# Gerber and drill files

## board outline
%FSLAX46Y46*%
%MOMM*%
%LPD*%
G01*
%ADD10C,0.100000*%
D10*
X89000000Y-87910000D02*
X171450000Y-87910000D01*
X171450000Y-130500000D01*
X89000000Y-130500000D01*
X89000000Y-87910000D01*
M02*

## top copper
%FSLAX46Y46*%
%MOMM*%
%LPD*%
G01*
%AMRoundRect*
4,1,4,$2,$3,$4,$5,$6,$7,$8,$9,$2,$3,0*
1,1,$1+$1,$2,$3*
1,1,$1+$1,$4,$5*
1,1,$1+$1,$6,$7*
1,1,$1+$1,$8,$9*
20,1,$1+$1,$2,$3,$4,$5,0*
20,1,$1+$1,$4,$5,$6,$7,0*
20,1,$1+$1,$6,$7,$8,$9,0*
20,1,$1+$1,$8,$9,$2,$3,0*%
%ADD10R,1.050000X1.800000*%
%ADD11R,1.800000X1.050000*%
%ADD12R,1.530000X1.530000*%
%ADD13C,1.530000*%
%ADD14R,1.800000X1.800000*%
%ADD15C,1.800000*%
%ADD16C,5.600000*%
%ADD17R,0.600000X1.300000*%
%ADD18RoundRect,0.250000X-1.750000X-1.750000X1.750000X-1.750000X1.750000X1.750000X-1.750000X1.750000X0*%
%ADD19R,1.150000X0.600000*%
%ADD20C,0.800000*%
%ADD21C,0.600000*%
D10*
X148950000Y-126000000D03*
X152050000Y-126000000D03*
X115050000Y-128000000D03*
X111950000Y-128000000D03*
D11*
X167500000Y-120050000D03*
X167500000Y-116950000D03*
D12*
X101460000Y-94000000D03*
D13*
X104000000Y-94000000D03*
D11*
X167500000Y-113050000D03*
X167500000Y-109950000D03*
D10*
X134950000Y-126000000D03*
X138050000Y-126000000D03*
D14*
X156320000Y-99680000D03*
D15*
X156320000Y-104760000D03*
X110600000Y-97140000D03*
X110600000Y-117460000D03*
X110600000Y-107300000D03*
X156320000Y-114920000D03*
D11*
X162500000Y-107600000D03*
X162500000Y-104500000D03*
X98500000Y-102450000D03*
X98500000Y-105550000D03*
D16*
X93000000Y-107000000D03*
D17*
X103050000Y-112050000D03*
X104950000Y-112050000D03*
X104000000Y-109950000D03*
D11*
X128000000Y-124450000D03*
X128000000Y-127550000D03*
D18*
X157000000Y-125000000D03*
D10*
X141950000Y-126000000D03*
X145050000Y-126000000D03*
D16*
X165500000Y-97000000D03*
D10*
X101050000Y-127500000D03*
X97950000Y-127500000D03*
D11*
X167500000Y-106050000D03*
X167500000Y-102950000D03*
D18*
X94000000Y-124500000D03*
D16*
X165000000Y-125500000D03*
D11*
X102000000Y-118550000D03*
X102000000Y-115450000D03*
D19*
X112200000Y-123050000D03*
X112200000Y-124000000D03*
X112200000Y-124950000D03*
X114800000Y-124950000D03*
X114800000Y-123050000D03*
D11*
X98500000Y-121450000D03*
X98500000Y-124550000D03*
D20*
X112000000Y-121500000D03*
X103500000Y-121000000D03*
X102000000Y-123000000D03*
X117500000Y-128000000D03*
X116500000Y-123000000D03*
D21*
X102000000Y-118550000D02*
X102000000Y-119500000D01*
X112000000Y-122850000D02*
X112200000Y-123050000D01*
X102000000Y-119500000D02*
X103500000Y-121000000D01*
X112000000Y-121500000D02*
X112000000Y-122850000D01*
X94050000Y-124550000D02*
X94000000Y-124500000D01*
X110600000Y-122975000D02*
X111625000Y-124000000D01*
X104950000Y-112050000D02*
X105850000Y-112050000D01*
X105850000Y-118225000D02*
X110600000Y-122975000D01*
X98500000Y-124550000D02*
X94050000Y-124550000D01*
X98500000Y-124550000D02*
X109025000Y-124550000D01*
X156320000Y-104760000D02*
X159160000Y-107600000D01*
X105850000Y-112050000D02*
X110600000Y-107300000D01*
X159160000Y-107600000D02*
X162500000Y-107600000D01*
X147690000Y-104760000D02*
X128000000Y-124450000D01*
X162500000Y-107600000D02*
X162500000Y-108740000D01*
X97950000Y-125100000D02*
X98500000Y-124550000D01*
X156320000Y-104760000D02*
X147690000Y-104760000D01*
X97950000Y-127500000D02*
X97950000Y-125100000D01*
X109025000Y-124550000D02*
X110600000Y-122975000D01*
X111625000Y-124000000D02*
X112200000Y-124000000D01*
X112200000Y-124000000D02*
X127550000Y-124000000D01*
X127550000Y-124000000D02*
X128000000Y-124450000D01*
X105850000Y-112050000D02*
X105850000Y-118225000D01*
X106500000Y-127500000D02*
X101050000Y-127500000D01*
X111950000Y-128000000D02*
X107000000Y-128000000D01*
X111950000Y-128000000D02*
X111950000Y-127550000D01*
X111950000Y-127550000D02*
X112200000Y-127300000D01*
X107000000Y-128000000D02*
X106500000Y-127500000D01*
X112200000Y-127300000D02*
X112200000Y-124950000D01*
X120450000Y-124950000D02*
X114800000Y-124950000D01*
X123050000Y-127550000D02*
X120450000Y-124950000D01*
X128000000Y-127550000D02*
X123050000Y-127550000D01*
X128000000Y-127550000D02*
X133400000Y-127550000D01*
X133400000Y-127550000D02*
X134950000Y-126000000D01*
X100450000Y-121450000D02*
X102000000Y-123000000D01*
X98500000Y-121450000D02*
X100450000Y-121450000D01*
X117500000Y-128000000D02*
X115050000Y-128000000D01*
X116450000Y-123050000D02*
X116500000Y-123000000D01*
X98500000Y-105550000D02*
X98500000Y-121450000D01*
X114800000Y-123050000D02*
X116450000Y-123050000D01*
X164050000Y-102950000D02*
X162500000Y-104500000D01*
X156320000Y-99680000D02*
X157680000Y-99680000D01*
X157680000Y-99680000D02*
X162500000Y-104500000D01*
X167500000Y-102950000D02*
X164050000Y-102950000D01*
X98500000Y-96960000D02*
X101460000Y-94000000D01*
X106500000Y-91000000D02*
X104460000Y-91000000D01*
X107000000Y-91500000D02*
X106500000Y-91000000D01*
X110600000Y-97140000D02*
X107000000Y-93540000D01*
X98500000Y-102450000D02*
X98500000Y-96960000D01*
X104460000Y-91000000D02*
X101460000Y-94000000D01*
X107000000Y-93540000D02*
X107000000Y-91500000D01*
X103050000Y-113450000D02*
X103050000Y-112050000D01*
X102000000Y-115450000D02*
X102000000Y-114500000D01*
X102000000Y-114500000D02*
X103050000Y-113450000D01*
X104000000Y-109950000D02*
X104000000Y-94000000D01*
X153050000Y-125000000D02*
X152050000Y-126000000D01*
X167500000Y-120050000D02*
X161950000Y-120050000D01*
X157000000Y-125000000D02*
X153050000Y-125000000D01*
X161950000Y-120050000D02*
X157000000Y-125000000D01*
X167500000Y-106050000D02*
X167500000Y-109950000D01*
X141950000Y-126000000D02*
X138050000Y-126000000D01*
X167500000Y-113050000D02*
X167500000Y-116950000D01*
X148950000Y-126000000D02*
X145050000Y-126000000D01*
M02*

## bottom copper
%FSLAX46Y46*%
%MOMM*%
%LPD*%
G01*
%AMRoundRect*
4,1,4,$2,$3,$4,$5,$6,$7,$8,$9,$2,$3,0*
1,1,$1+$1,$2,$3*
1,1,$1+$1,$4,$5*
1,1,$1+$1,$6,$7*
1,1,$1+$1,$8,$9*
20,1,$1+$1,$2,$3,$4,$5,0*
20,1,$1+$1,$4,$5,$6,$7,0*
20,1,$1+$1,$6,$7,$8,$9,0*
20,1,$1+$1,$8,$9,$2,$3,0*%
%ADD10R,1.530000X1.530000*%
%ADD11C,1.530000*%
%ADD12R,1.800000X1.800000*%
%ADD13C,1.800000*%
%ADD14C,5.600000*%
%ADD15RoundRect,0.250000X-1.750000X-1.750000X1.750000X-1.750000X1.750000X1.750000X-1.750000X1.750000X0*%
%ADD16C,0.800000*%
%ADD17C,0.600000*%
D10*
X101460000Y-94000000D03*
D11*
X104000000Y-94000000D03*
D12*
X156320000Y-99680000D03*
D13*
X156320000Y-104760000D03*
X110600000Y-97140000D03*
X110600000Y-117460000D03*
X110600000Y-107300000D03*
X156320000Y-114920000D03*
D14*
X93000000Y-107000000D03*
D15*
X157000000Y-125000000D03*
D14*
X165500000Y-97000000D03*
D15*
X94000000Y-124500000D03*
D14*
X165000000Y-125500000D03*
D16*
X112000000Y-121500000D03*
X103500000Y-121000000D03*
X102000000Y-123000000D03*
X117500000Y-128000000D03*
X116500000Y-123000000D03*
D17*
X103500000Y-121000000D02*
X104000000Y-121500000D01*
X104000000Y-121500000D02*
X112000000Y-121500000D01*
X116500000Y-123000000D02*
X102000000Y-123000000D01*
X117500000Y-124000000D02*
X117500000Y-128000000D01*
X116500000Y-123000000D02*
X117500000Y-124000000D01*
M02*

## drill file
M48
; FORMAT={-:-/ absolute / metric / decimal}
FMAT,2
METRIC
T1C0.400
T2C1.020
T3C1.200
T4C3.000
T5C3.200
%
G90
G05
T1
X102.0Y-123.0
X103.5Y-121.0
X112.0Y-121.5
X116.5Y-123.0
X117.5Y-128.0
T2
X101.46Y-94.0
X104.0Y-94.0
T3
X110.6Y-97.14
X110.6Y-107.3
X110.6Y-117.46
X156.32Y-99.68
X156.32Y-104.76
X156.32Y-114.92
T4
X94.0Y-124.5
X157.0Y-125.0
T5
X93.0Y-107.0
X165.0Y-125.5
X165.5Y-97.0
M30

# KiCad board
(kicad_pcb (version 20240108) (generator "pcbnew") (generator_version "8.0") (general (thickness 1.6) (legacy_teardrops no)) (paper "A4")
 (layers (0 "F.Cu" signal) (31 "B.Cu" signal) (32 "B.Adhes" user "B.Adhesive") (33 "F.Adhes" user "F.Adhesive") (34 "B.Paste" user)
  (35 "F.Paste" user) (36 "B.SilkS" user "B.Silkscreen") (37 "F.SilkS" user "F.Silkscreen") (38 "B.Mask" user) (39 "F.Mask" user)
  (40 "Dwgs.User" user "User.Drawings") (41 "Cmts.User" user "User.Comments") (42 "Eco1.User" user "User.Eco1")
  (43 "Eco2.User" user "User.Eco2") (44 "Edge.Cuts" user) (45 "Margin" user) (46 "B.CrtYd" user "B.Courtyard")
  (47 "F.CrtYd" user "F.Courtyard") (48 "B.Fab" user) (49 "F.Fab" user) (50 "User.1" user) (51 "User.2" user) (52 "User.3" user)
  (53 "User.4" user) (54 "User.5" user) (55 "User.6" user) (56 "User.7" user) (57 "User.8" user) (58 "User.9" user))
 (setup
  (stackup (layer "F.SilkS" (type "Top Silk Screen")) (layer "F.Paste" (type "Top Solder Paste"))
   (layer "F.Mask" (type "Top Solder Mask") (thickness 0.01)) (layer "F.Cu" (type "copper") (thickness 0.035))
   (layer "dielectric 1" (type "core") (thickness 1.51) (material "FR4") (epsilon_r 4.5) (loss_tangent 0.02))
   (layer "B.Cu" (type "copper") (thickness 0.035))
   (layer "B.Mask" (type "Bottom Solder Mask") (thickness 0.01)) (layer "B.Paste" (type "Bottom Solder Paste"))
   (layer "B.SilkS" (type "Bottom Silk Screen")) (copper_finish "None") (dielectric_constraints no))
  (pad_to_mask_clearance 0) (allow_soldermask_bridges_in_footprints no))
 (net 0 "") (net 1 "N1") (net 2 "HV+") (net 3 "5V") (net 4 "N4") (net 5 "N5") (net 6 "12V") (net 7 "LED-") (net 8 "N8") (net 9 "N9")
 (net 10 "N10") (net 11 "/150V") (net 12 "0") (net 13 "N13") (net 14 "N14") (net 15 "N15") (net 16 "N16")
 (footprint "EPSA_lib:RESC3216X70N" (layer "F.Cu") (at 150.5 126)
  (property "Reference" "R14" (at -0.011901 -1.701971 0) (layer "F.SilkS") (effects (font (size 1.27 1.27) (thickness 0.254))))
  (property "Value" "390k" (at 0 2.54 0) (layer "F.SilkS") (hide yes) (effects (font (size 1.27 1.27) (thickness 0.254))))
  (pad "1" smd rect (at -1.55 0) (size 1.05 1.8) (layers "F.Cu" "F.Paste" "F.Mask") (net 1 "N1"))
  (pad "2" smd rect (at 1.55 0) (size 1.05 1.8) (layers "F.Cu" "F.Paste" "F.Mask") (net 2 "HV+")))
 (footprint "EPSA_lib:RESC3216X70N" (layer "F.Cu") (at 113.5 128 180)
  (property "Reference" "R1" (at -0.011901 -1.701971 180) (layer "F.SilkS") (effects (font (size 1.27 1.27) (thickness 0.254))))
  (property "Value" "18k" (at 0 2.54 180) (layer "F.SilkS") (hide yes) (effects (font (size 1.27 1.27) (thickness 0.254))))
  (pad "1" smd rect (at -1.55 0 180) (size 1.05 1.8) (layers "F.Cu" "F.Paste" "F.Mask") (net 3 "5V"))
  (pad "2" smd rect (at 1.55 0 180) (size 1.05 1.8) (layers "F.Cu" "F.Paste" "F.Mask") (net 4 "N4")))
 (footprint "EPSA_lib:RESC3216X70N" (layer "F.Cu") (at 167.5 118.5 90)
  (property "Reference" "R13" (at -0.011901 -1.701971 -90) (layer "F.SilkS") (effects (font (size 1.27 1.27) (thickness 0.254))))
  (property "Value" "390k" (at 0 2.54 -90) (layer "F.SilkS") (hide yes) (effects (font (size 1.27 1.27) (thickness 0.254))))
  (pad "1" smd rect (at -1.55 0 90) (size 1.05 1.8) (layers "F.Cu" "F.Paste" "F.Mask") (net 2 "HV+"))
  (pad "2" smd rect (at 1.55 0 90) (size 1.05 1.8) (layers "F.Cu" "F.Paste" "F.Mask") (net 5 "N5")))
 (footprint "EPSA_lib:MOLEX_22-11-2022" (layer "F.Cu") (at 101.46 94)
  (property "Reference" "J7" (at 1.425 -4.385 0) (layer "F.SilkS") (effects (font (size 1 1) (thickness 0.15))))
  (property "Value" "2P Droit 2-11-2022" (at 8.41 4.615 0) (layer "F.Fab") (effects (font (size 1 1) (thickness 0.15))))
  (pad "1" thru_hole rect (at 0 0) (size 1.53 1.53) (drill 1.02) (layers "*.Cu" "*.Mask") (remove_unused_layers no) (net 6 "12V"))
  (pad "2" thru_hole circle (at 2.54 0) (size 1.53 1.53) (drill 1.02) (layers "*.Cu" "*.Mask") (remove_unused_layers no) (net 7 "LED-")))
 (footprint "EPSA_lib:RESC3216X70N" (layer "F.Cu") (at 167.5 111.5 90)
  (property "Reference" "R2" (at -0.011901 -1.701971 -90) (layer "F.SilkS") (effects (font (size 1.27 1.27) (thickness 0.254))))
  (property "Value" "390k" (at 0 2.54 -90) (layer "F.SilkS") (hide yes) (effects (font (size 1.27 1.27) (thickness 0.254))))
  (pad "1" smd rect (at -1.55 0 90) (size 1.05 1.8) (layers "F.Cu" "F.Paste" "F.Mask") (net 5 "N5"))
  (pad "2" smd rect (at 1.55 0 90) (size 1.05 1.8) (layers "F.Cu" "F.Paste" "F.Mask") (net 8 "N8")))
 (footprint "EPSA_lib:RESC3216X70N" (layer "F.Cu") (at 136.5 126)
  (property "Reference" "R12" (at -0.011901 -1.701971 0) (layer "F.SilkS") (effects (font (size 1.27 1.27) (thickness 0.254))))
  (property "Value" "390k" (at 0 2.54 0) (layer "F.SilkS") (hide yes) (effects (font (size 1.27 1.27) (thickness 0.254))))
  (pad "1" smd rect (at -1.55 0) (size 1.05 1.8) (layers "F.Cu" "F.Paste" "F.Mask") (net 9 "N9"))
  (pad "2" smd rect (at 1.55 0) (size 1.05 1.8) (layers "F.Cu" "F.Paste" "F.Mask") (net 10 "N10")))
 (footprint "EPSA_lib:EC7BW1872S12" (layer "F.Cu") (at 140.82 130.18 180)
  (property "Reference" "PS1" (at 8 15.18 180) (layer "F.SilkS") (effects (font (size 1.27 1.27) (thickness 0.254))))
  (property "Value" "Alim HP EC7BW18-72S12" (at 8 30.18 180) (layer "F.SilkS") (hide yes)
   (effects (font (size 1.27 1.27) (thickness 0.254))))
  (pad "1" thru_hole rect (at -15.5 30.5 270) (size 1.8 1.8) (drill 1.2) (layers "*.Cu" "*.Mask") (remove_unused_layers no) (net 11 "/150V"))
  (pad "2" thru_hole circle (at -15.5 25.42 270) (size 1.8 1.8) (drill 1.2) (layers "*.Cu" "*.Mask") (remove_unused_layers no) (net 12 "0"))
  (pad "3" thru_hole circle (at 30.22 33.04 270) (size 1.8 1.8) (drill 1.2) (layers "*.Cu" "*.Mask") (remove_unused_layers no) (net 6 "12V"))
  (pad "4" thru_hole circle (at 30.22 12.72 270) (size 1.8 1.8) (drill 1.2) (layers "*.Cu" "*.Mask") (remove_unused_layers no)
   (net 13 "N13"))
  (pad "5" thru_hole circle (at 30.22 22.88 270) (size 1.8 1.8) (drill 1.2) (layers "*.Cu" "*.Mask") (remove_unused_layers no) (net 12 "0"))
  (pad "6" thru_hole circle (at -15.5 15.26 270) (size 1.8 1.8) (drill 1.2) (layers "*.Cu" "*.Mask") (remove_unused_layers no)
   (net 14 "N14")))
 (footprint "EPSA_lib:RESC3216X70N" (layer "F.Cu") (at 162.5 106.05 90)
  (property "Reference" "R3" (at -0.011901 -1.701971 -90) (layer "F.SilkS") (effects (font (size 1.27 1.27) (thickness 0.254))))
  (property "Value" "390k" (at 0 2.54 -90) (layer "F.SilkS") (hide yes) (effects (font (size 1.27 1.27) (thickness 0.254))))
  (pad "1" smd rect (at -1.55 0 90) (size 1.05 1.8) (layers "F.Cu" "F.Paste" "F.Mask") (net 12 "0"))
  (pad "2" smd rect (at 1.55 0 90) (size 1.05 1.8) (layers "F.Cu" "F.Paste" "F.Mask") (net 11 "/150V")))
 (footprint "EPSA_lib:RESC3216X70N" (layer "F.Cu") (at 98.5 104 -90)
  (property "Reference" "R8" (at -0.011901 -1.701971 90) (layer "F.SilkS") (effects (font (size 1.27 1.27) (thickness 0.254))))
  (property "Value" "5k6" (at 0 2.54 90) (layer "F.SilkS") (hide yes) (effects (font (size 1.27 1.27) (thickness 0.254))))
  (pad "1" smd rect (at -1.55 0 270) (size 1.05 1.8) (layers "F.Cu" "F.Paste" "F.Mask") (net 6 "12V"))
  (pad "2" smd rect (at 1.55 0 270) (size 1.05 1.8) (layers "F.Cu" "F.Paste" "F.Mask") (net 3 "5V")))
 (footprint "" (layer "F.Cu") (at 93 107)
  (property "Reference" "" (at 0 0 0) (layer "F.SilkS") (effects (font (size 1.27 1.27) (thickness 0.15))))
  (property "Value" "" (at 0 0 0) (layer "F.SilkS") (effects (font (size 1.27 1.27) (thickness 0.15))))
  (pad "1" thru_hole circle (at 0 0) (size 5.6 5.6) (drill 3.2) (layers "*.Cu" "*.Mask") (remove_unused_layers no)))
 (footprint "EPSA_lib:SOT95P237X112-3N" (layer "F.Cu") (at 104 111 90)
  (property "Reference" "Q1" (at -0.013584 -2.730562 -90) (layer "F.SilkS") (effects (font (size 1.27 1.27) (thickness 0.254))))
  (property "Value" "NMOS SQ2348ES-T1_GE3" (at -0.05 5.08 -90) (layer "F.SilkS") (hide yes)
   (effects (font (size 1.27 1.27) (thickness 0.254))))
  (pad "1" smd rect (at -1.05 -0.95 180) (size 0.6 1.3) (layers "F.Cu" "F.Paste" "F.Mask") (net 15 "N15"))
  (pad "2" smd rect (at -1.05 0.95 180) (size 0.6 1.3) (layers "F.Cu" "F.Paste" "F.Mask") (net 12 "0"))
  (pad "3" smd rect (at 1.05 0 180) (size 0.6 1.3) (layers "F.Cu" "F.Paste" "F.Mask") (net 7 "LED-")))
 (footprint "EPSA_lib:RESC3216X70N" (layer "F.Cu") (at 128 126 -90)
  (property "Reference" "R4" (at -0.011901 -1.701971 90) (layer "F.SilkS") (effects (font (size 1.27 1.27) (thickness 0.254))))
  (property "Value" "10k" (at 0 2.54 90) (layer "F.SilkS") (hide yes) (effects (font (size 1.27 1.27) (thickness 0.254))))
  (pad "1" smd rect (at -1.55 0 270) (size 1.05 1.8) (layers "F.Cu" "F.Paste" "F.Mask") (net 12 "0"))
  (pad "2" smd rect (at 1.55 0 270) (size 1.05 1.8) (layers "F.Cu" "F.Paste" "F.Mask") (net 9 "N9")))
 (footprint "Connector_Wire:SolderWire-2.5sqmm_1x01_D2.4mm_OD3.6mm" (layer "F.Cu") (at 157 125)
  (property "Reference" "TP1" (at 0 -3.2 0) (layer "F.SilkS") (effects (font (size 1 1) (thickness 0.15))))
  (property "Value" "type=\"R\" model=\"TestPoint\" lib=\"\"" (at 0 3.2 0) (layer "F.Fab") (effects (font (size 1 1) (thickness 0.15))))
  (pad "1" thru_hole roundrect (at 0 0) (size 4 4) (drill 3) (layers "*.Cu" "*.Mask") (remove_unused_layers no) (roundrect_rratio 0.0625)
   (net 2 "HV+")))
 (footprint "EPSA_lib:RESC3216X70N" (layer "F.Cu") (at 143.5 126)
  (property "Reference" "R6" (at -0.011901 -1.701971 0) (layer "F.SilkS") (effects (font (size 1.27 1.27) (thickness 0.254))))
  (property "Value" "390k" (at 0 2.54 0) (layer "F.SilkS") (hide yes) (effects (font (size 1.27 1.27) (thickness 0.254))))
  (pad "1" smd rect (at -1.55 0) (size 1.05 1.8) (layers "F.Cu" "F.Paste" "F.Mask") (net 10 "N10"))
  (pad "2" smd rect (at 1.55 0) (size 1.05 1.8) (layers "F.Cu" "F.Paste" "F.Mask") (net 1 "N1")))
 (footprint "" (layer "F.Cu") (at 165.5 97)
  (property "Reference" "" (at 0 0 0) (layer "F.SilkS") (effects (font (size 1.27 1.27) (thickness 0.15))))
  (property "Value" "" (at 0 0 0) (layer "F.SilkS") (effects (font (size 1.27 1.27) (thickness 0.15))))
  (pad "1" thru_hole circle (at 0 0) (size 5.6 5.6) (drill 3.2) (layers "*.Cu" "*.Mask") (remove_unused_layers no)))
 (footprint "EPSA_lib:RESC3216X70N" (layer "F.Cu") (at 99.5 127.5 180)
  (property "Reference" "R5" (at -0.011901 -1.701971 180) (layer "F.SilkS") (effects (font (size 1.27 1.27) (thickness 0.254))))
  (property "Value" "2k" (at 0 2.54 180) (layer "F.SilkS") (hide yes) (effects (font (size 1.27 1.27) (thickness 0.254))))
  (pad "1" smd rect (at -1.55 0 180) (size 1.05 1.8) (layers "F.Cu" "F.Paste" "F.Mask") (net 4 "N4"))
  (pad "2" smd rect (at 1.55 0 180) (size 1.05 1.8) (layers "F.Cu" "F.Paste" "F.Mask") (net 12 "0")))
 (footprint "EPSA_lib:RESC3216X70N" (layer "F.Cu") (at 167.5 104.5 90)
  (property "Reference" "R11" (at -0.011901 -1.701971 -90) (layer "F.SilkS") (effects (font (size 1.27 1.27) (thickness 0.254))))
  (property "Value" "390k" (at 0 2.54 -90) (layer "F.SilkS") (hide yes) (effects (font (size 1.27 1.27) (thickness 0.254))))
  (pad "1" smd rect (at -1.55 0 90) (size 1.05 1.8) (layers "F.Cu" "F.Paste" "F.Mask") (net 8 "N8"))
  (pad "2" smd rect (at 1.55 0 90) (size 1.05 1.8) (layers "F.Cu" "F.Paste" "F.Mask") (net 11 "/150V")))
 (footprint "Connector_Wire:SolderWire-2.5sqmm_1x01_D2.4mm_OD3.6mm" (layer "F.Cu") (at 94 124.5)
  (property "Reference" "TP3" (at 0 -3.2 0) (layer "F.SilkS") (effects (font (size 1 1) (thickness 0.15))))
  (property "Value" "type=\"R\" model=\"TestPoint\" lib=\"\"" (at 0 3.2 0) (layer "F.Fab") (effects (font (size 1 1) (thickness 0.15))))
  (pad "1" thru_hole roundrect (at 0 0) (size 4 4) (drill 3) (layers "*.Cu" "*.Mask") (remove_unused_layers no) (roundrect_rratio 0.0625)
   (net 12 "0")))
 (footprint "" (layer "F.Cu") (at 165 125.5)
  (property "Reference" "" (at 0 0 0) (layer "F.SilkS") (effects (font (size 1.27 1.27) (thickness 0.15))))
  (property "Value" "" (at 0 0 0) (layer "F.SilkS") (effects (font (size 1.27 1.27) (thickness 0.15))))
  (pad "1" thru_hole circle (at 0 0) (size 5.6 5.6) (drill 3.2) (layers "*.Cu" "*.Mask") (remove_unused_layers no)))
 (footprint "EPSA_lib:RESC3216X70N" (layer "F.Cu") (at 102 117 90)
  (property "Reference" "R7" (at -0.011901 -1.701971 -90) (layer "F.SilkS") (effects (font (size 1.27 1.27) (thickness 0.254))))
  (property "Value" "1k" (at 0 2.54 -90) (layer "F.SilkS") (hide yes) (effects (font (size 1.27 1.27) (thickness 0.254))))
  (pad "1" smd rect (at -1.55 0 90) (size 1.05 1.8) (layers "F.Cu" "F.Paste" "F.Mask") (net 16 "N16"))
  (pad "2" smd rect (at 1.55 0 90) (size 1.05 1.8) (layers "F.Cu" "F.Paste" "F.Mask") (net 15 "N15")))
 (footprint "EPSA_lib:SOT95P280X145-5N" (layer "F.Cu") (at 113.5 124)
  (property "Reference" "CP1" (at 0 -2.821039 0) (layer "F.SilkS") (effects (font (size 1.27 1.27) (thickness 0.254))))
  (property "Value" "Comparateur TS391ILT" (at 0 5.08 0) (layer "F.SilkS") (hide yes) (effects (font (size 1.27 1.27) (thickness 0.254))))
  (pad "1" smd rect (at -1.3 -0.95 90) (size 0.6 1.15) (layers "F.Cu" "F.Paste" "F.Mask") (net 16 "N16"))
  (pad "2" smd rect (at -1.3 0 90) (size 0.6 1.15) (layers "F.Cu" "F.Paste" "F.Mask") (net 12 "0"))
  (pad "3" smd rect (at -1.3 0.95 90) (size 0.6 1.15) (layers "F.Cu" "F.Paste" "F.Mask") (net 4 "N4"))
  (pad "4" smd rect (at 1.3 0.95 90) (size 0.6 1.15) (layers "F.Cu" "F.Paste" "F.Mask") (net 9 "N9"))
  (pad "5" smd rect (at 1.3 -0.95 90) (size 0.6 1.15) (layers "F.Cu" "F.Paste" "F.Mask") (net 3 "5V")))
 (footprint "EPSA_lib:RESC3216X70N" (layer "F.Cu") (at 98.5 123 -90)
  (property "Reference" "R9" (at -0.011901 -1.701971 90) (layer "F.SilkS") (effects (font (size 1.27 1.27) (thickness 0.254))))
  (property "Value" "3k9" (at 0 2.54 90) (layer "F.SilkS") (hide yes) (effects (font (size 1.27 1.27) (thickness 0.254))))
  (pad "1" smd rect (at -1.55 0 270) (size 1.05 1.8) (layers "F.Cu" "F.Paste" "F.Mask") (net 3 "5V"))
  (pad "2" smd rect (at 1.55 0 270) (size 1.05 1.8) (layers "F.Cu" "F.Paste" "F.Mask") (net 12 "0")))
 (gr_rect (start 89 87.91) (end 171.45 130.5) (stroke (width 0.1) (type default)) (fill none) (layer "Edge.Cuts"))
 (segment (start 102 118.55) (end 102 119.5) (width 0.6) (layer "F.Cu") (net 16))
 (segment (start 112 122.85) (end 112.2 123.05) (width 0.6) (layer "F.Cu") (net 16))
 (segment (start 102 119.5) (end 103.5 121) (width 0.6) (layer "F.Cu") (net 16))
 (segment (start 112 121.5) (end 112 122.85) (width 0.6) (layer "F.Cu") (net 16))
 (via (at 112 121.5) (size 0.8) (drill 0.4) (layers "F.Cu" "B.Cu") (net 16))
 (via (at 103.5 121) (size 0.8) (drill 0.4) (layers "F.Cu" "B.Cu") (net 16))
 (segment (start 103.5 121) (end 104 121.5) (width 0.6) (layer "B.Cu") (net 16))
 (segment (start 104 121.5) (end 112 121.5) (width 0.6) (layer "B.Cu") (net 16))
 (segment (start 94.05 124.55) (end 94 124.5) (width 0.6) (layer "F.Cu") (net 12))
 (segment (start 110.6 122.975) (end 111.625 124) (width 0.6) (layer "F.Cu") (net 12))
 (segment (start 104.95 112.05) (end 105.85 112.05) (width 0.6) (layer "F.Cu") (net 12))
 (segment (start 105.85 118.225) (end 110.6 122.975) (width 0.6) (layer "F.Cu") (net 12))
 (segment (start 98.5 124.55) (end 94.05 124.55) (width 0.6) (layer "F.Cu") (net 12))
 (segment (start 98.5 124.55) (end 109.025 124.55) (width 0.6) (layer "F.Cu") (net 12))
 (segment (start 156.32 104.76) (end 159.16 107.6) (width 0.6) (layer "F.Cu") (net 12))
 (segment (start 105.85 112.05) (end 110.6 107.3) (width 0.6) (layer "F.Cu") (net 12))
 (segment (start 159.16 107.6) (end 162.5 107.6) (width 0.6) (layer "F.Cu") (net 12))
 (segment (start 147.69 104.76) (end 128 124.45) (width 0.6) (layer "F.Cu") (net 12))
 (segment (start 162.5 107.6) (end 162.5 108.74) (width 0.6) (layer "F.Cu") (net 12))
 (segment (start 97.95 125.1) (end 98.5 124.55) (width 0.6) (layer "F.Cu") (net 12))
 (segment (start 156.32 104.76) (end 147.69 104.76) (width 0.6) (layer "F.Cu") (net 12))
 (segment (start 97.95 127.5) (end 97.95 125.1) (width 0.6) (layer "F.Cu") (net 12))
 (segment (start 109.025 124.55) (end 110.6 122.975) (width 0.6) (layer "F.Cu") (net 12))
 (segment (start 111.625 124) (end 112.2 124) (width 0.6) (layer "F.Cu") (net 12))
 (segment (start 112.2 124) (end 127.55 124) (width 0.6) (layer "F.Cu") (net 12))
 (segment (start 127.55 124) (end 128 124.45) (width 0.6) (layer "F.Cu") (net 12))
 (segment (start 105.85 112.05) (end 105.85 118.225) (width 0.6) (layer "F.Cu") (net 12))
 (segment (start 106.5 127.5) (end 101.05 127.5) (width 0.6) (layer "F.Cu") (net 4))
 (segment (start 111.95 128) (end 107 128) (width 0.6) (layer "F.Cu") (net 4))
 (segment (start 111.95 128) (end 111.95 127.55) (width 0.6) (layer "F.Cu") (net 4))
 (segment (start 111.95 127.55) (end 112.2 127.3) (width 0.6) (layer "F.Cu") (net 4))
 (segment (start 107 128) (end 106.5 127.5) (width 0.6) (layer "F.Cu") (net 4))
 (segment (start 112.2 127.3) (end 112.2 124.95) (width 0.6) (layer "F.Cu") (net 4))
 (segment (start 120.45 124.95) (end 114.8 124.95) (width 0.6) (layer "F.Cu") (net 9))
 (segment (start 123.05 127.55) (end 120.45 124.95) (width 0.6) (layer "F.Cu") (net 9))
 (segment (start 128 127.55) (end 123.05 127.55) (width 0.6) (layer "F.Cu") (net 9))
 (segment (start 128 127.55) (end 133.4 127.55) (width 0.6) (layer "F.Cu") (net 9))
 (segment (start 133.4 127.55) (end 134.95 126) (width 0.6) (layer "F.Cu") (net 9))
 (segment (start 100.45 121.45) (end 102 123) (width 0.6) (layer "F.Cu") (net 3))
 (segment (start 98.5 121.45) (end 100.45 121.45) (width 0.6) (layer "F.Cu") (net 3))
 (segment (start 117.5 128) (end 115.05 128) (width 0.6) (layer "F.Cu") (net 3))
 (segment (start 116.45 123.05) (end 116.5 123) (width 0.6) (layer "F.Cu") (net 3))
 (segment (start 98.5 105.55) (end 98.5 121.45) (width 0.6) (layer "F.Cu") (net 3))
 (segment (start 114.8 123.05) (end 116.45 123.05) (width 0.6) (layer "F.Cu") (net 3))
 (via (at 102 123) (size 0.8) (drill 0.4) (layers "F.Cu" "B.Cu") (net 3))
 (via (at 117.5 128) (size 0.8) (drill 0.4) (layers "F.Cu" "B.Cu") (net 3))
 (via (at 116.5 123) (size 0.8) (drill 0.4) (layers "F.Cu" "B.Cu") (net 3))
 (segment (start 116.5 123) (end 102 123) (width 0.6) (layer "B.Cu") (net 3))
 (segment (start 117.5 124) (end 117.5 128) (width 0.6) (layer "B.Cu") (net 3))
 (segment (start 116.5 123) (end 117.5 124) (width 0.6) (layer "B.Cu") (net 3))
 (segment (start 164.05 102.95) (end 162.5 104.5) (width 0.6) (layer "F.Cu") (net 11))
 (segment (start 156.32 99.68) (end 157.68 99.68) (width 0.6) (layer "F.Cu") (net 11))
 (segment (start 157.68 99.68) (end 162.5 104.5) (width 0.6) (layer "F.Cu") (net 11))
 (segment (start 167.5 102.95) (end 164.05 102.95) (width 0.6) (layer "F.Cu") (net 11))
 (segment (start 98.5 96.96) (end 101.46 94) (width 0.6) (layer "F.Cu") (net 6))
 (segment (start 106.5 91) (end 104.46 91) (width 0.6) (layer "F.Cu") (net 6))
 (segment (start 107 91.5) (end 106.5 91) (width 0.6) (layer "F.Cu") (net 6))
 (segment (start 110.6 97.14) (end 107 93.54) (width 0.6) (layer "F.Cu") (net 6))
 (segment (start 98.5 102.45) (end 98.5 96.96) (width 0.6) (layer "F.Cu") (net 6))
 (segment (start 104.46 91) (end 101.46 94) (width 0.6) (layer "F.Cu") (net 6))
 (segment (start 107 93.54) (end 107 91.5) (width 0.6) (layer "F.Cu") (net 6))
 (segment (start 103.05 113.45) (end 103.05 112.05) (width 0.6) (layer "F.Cu") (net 15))
 (segment (start 102 115.45) (end 102 114.5) (width 0.6) (layer "F.Cu") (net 15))
 (segment (start 102 114.5) (end 103.05 113.45) (width 0.6) (layer "F.Cu") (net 15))
 (segment (start 104 109.95) (end 104 94) (width 0.6) (layer "F.Cu") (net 7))
 (segment (start 153.05 125) (end 152.05 126) (width 0.6) (layer "F.Cu") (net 2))
 (segment (start 167.5 120.05) (end 161.95 120.05) (width 0.6) (layer "F.Cu") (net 2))
 (segment (start 157 125) (end 153.05 125) (width 0.6) (layer "F.Cu") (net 2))
 (segment (start 161.95 120.05) (end 157 125) (width 0.6) (layer "F.Cu") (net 2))
 (segment (start 167.5 106.05) (end 167.5 109.95) (width 0.6) (layer "F.Cu") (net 8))
 (segment (start 141.95 126) (end 138.05 126) (width 0.6) (layer "F.Cu") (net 10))
 (segment (start 167.5 113.05) (end 167.5 116.95) (width 0.6) (layer "F.Cu") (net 5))
 (segment (start 148.95 126) (end 145.05 126) (width 0.6) (layer "F.Cu") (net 1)))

